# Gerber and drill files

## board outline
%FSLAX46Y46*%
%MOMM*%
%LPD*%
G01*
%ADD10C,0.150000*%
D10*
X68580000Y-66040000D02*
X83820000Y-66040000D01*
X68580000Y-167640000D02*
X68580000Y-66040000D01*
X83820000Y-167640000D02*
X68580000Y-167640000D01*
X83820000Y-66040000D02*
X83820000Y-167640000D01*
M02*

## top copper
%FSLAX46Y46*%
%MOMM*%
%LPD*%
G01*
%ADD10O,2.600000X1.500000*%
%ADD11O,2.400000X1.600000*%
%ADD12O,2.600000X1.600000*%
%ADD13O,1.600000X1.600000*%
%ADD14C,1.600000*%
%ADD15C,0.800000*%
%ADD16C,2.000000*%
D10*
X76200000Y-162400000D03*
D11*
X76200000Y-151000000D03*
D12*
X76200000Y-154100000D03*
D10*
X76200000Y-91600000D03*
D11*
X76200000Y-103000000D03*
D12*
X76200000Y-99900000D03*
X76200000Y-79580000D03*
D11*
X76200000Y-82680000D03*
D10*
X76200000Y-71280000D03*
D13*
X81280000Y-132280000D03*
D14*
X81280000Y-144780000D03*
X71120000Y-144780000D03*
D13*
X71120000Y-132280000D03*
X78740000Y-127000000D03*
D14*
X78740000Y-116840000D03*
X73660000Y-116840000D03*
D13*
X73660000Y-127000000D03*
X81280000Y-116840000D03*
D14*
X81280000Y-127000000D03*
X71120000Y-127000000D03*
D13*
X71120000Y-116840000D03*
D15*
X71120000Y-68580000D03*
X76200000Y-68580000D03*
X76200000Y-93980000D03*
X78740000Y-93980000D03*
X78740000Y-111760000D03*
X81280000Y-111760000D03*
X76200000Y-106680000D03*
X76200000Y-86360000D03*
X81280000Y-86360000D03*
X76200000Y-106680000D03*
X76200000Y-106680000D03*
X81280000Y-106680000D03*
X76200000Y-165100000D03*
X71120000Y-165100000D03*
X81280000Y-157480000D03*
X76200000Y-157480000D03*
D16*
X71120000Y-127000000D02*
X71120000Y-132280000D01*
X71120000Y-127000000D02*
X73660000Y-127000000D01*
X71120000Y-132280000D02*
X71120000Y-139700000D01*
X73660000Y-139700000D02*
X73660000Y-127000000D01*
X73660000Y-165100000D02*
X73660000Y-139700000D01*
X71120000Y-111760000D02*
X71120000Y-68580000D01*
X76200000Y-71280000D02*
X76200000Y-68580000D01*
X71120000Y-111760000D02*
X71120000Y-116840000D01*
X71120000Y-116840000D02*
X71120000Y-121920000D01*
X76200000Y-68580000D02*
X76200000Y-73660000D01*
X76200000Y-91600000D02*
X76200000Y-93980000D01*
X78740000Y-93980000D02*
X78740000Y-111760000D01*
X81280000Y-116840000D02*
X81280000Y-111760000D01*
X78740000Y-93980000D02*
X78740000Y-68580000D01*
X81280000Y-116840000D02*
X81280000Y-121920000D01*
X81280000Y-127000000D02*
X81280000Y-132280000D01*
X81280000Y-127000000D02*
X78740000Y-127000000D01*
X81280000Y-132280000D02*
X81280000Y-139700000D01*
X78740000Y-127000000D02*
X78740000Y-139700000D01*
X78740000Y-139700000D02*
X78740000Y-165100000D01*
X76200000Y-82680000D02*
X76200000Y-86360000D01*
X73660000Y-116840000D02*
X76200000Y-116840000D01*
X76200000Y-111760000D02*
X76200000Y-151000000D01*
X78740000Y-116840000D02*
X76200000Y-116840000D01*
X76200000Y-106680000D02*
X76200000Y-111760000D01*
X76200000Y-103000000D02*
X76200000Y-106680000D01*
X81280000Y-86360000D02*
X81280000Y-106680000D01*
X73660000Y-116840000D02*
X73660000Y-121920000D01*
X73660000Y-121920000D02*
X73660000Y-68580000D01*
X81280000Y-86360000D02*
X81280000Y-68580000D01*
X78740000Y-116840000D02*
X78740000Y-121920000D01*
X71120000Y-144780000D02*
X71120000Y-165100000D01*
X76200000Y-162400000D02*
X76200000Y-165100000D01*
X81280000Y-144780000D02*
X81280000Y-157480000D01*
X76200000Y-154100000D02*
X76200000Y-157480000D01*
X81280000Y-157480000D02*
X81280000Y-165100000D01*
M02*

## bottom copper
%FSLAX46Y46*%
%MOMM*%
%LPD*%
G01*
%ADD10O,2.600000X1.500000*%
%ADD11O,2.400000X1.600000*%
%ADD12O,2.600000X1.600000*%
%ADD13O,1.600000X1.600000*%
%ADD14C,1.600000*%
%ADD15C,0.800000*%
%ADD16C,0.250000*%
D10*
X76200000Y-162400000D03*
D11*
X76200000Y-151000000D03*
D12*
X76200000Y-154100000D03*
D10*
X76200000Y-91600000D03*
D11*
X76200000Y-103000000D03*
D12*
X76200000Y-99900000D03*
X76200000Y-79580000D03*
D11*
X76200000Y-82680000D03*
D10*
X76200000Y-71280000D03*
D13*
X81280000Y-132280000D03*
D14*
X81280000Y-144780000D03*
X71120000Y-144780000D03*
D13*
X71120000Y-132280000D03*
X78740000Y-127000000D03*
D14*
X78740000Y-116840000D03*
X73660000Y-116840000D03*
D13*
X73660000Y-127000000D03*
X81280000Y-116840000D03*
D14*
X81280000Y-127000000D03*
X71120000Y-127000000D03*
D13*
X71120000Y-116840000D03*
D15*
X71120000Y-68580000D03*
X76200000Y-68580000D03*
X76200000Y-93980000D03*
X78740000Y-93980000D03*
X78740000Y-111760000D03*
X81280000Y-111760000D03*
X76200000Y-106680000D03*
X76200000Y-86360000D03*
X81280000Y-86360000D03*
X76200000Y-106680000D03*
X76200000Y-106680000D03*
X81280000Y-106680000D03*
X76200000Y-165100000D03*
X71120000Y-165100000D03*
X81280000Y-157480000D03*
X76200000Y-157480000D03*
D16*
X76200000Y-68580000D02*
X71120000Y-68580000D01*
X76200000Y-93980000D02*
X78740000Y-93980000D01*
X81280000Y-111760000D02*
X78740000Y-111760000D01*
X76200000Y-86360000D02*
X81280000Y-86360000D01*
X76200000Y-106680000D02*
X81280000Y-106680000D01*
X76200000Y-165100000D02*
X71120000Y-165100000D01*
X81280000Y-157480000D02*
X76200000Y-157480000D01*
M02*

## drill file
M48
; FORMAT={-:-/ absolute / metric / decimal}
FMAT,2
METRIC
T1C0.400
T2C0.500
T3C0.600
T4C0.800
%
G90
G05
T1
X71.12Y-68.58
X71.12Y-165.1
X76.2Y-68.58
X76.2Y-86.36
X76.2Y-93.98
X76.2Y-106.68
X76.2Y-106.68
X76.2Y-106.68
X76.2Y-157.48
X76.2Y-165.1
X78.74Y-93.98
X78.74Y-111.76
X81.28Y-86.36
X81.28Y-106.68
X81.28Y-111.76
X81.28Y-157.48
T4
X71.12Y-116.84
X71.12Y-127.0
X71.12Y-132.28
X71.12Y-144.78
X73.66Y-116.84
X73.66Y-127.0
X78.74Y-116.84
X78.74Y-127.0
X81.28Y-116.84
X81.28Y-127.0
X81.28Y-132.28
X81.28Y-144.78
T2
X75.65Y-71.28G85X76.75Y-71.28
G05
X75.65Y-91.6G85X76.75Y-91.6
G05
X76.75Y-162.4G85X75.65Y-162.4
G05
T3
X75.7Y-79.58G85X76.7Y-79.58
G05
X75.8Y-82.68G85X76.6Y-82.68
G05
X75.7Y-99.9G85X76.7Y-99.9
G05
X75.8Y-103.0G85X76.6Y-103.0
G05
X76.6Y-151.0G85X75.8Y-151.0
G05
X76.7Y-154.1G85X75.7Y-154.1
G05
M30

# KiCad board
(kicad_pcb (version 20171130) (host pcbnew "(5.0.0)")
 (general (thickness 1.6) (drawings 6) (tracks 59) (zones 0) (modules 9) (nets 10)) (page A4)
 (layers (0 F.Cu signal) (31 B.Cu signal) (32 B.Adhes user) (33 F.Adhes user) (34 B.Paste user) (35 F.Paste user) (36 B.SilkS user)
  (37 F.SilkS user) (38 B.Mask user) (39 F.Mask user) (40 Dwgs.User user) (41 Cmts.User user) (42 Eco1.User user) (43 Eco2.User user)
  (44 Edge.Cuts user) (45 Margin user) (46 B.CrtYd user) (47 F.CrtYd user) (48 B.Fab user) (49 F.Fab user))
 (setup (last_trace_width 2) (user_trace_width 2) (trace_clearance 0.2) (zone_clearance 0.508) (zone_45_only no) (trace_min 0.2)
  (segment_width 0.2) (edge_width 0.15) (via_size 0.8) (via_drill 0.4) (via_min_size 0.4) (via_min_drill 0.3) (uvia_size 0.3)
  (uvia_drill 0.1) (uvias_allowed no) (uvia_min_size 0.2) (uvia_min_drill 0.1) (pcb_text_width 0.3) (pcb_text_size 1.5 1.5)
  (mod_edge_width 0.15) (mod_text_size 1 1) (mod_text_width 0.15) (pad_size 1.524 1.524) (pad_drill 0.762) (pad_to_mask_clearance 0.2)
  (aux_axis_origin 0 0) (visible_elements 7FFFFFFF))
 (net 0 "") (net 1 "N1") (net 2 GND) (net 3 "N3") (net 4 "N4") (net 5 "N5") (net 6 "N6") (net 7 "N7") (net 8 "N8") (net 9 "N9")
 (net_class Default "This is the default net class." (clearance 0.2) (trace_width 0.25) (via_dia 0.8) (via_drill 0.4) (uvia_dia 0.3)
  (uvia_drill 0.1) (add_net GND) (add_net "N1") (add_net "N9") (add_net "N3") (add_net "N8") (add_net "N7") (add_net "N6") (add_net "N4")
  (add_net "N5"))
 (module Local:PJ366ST (layer F.Cu) (at 76.2 157.48 180)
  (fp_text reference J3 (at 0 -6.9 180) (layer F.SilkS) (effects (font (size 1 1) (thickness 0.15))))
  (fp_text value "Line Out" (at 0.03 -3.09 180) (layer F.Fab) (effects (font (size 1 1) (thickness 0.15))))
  (pad T thru_hole oval (at 0 -4.92 180) (size 2.6 1.5) (drill oval 1.6 0.5) (layers *.Cu *.Mask) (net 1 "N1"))
  (pad S thru_hole oval (at 0 6.48 180) (size 2.4 1.6) (drill oval 1.4 0.6) (layers *.Cu *.Mask) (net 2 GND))
  (pad R thru_hole oval (at 0 3.38 180) (size 2.6 1.6) (drill oval 1.6 0.6) (layers *.Cu *.Mask) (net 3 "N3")))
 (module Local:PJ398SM (layer F.Cu) (at 76.2 96.52)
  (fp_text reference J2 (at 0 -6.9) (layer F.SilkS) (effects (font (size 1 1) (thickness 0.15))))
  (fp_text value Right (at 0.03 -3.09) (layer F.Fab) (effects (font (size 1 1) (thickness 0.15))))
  (pad T thru_hole oval (at 0 -4.92) (size 2.6 1.5) (drill oval 1.6 0.5) (layers *.Cu *.Mask) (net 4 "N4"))
  (pad S thru_hole oval (at 0 6.48) (size 2.4 1.6) (drill oval 1.4 0.6) (layers *.Cu *.Mask) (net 2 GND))
  (pad TN thru_hole oval (at 0 3.38) (size 2.6 1.6) (drill oval 1.6 0.6) (layers *.Cu *.Mask) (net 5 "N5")))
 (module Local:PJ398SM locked (layer F.Cu) (at 76.2 76.2)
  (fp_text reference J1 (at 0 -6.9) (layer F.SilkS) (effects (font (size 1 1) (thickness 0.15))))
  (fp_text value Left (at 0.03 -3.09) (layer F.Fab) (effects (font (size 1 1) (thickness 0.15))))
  (pad TN thru_hole oval (at 0 3.38) (size 2.6 1.6) (drill oval 1.6 0.6) (layers *.Cu *.Mask) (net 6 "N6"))
  (pad S thru_hole oval (at 0 6.48) (size 2.4 1.6) (drill oval 1.4 0.6) (layers *.Cu *.Mask) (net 2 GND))
  (pad T thru_hole oval (at 0 -4.92) (size 2.6 1.5) (drill oval 1.6 0.5) (layers *.Cu *.Mask) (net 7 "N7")))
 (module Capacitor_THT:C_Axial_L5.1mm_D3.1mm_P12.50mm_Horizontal (layer F.Cu) (at 81.28 144.78 90)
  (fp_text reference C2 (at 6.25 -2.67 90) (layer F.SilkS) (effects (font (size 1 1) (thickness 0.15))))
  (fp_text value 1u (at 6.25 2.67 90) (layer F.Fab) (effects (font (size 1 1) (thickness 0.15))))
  (pad 2 thru_hole oval (at 12.5 0 90) (size 1.6 1.6) (drill 0.8) (layers *.Cu *.Mask) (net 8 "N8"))
  (pad 1 thru_hole circle (at 0 0 90) (size 1.6 1.6) (drill 0.8) (layers *.Cu *.Mask) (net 3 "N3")))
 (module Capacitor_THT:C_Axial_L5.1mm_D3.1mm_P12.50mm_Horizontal (layer F.Cu) (at 71.12 144.78 90)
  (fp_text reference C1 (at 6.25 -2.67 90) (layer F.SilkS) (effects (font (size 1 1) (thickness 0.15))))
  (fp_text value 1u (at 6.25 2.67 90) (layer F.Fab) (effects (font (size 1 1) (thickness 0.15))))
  (pad 1 thru_hole circle (at 0 0 90) (size 1.6 1.6) (drill 0.8) (layers *.Cu *.Mask) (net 1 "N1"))
  (pad 2 thru_hole oval (at 12.5 0 90) (size 1.6 1.6) (drill 0.8) (layers *.Cu *.Mask) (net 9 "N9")))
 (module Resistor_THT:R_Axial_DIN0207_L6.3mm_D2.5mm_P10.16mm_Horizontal (layer F.Cu) (at 78.74 116.84 270)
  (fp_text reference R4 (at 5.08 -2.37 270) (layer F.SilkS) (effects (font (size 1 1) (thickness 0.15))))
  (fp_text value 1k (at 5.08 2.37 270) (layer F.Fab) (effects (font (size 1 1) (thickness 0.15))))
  (pad 2 thru_hole oval (at 10.16 0 270) (size 1.6 1.6) (drill 0.8) (layers *.Cu *.Mask) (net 8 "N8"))
  (pad 1 thru_hole circle (at 0 0 270) (size 1.6 1.6) (drill 0.8) (layers *.Cu *.Mask) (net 2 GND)))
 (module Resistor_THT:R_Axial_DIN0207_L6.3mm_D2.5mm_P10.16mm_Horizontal (layer F.Cu) (at 73.66 116.84 270)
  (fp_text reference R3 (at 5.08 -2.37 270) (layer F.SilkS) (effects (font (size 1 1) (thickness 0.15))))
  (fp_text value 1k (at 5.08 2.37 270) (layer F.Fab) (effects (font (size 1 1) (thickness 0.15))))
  (pad 1 thru_hole circle (at 0 0 270) (size 1.6 1.6) (drill 0.8) (layers *.Cu *.Mask) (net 2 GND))
  (pad 2 thru_hole oval (at 10.16 0 270) (size 1.6 1.6) (drill 0.8) (layers *.Cu *.Mask) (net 9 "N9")))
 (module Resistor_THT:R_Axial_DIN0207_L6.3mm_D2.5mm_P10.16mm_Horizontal (layer F.Cu) (at 81.28 127 90)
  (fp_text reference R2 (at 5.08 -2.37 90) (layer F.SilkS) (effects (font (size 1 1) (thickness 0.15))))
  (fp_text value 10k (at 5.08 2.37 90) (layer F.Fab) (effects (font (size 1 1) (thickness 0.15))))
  (pad 2 thru_hole oval (at 10.16 0 90) (size 1.6 1.6) (drill 0.8) (layers *.Cu *.Mask) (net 4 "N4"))
  (pad 1 thru_hole circle (at 0 0 90) (size 1.6 1.6) (drill 0.8) (layers *.Cu *.Mask) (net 8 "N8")))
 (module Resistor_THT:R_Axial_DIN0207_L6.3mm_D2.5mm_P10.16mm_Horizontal (layer F.Cu) (at 71.12 127 90)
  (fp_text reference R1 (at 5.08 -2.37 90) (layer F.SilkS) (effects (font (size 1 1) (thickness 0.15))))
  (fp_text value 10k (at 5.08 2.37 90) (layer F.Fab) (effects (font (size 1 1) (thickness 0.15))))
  (pad 1 thru_hole circle (at 0 0 90) (size 1.6 1.6) (drill 0.8) (layers *.Cu *.Mask) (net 9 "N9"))
  (pad 2 thru_hole oval (at 10.16 0 90) (size 1.6 1.6) (drill 0.8) (layers *.Cu *.Mask) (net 7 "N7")))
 (gr_line (start 68.58 66.04) (end 83.82 66.04) (layer Edge.Cuts) (width 0.15))
 (gr_line (start 68.58 167.64) (end 68.58 66.04) (layer Edge.Cuts) (width 0.15))
 (gr_line (start 83.82 167.64) (end 68.58 167.64) (layer Edge.Cuts) (width 0.15))
 (gr_line (start 83.82 66.04) (end 83.82 167.64) (layer Edge.Cuts) (width 0.15))
 (segment (start 71.12 127) (end 71.12 132.28) (width 2) (layer F.Cu) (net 9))
 (segment (start 71.12 127) (end 73.66 127) (width 2) (layer F.Cu) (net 9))
 (segment (start 71.12 132.28) (end 71.12 139.7) (width 2) (layer F.Cu) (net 9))
 (segment (start 73.66 139.7) (end 73.66 127) (width 2) (layer F.Cu) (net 9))
 (segment (start 73.66 165.1) (end 73.66 139.7) (width 2) (layer F.Cu) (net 9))
 (segment (start 71.12 111.76) (end 71.12 68.58) (width 2) (layer F.Cu) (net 7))
 (via (at 71.12 68.58) (size 0.8) (drill 0.4) (layers F.Cu B.Cu) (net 7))
 (segment (start 76.2 71.28) (end 76.2 68.58) (width 2) (layer F.Cu) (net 7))
 (via (at 76.2 68.58) (size 0.8) (drill 0.4) (layers F.Cu B.Cu) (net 7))
 (segment (start 76.2 68.58) (end 71.12 68.58) (width 0.25) (layer B.Cu) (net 7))
 (segment (start 71.12 111.76) (end 71.12 116.84) (width 2) (layer F.Cu) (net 7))
 (segment (start 71.12 116.84) (end 71.12 121.92) (width 2) (layer F.Cu) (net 7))
 (segment (start 76.2 68.58) (end 76.2 73.66) (width 2) (layer F.Cu) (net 7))
 (segment (start 76.2 91.6) (end 76.2 93.98) (width 2) (layer F.Cu) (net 4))
 (via (at 76.2 93.98) (size 0.8) (drill 0.4) (layers F.Cu B.Cu) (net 4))
 (via (at 78.74 93.98) (size 0.8) (drill 0.4) (layers F.Cu B.Cu) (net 4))
 (segment (start 76.2 93.98) (end 78.74 93.98) (width 0.25) (layer B.Cu) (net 4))
 (segment (start 78.74 93.98) (end 78.74 111.76) (width 2) (layer F.Cu) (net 4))
 (via (at 78.74 111.76) (size 0.8) (drill 0.4) (layers F.Cu B.Cu) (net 4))
 (via (at 81.28 111.76) (size 0.8) (drill 0.4) (layers F.Cu B.Cu) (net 4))
 (segment (start 81.28 116.84) (end 81.28 111.76) (width 2) (layer F.Cu) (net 4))
 (segment (start 81.28 111.76) (end 78.74 111.76) (width 0.25) (layer B.Cu) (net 4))
 (segment (start 78.74 93.98) (end 78.74 68.58) (width 2) (layer F.Cu) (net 4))
 (segment (start 81.28 116.84) (end 81.28 121.92) (width 2) (layer F.Cu) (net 4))
 (segment (start 81.28 127) (end 81.28 132.28) (width 2) (layer F.Cu) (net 8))
 (segment (start 81.28 127) (end 78.74 127) (width 2) (layer F.Cu) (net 8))
 (segment (start 81.28 132.28) (end 81.28 139.7) (width 2) (layer F.Cu) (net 8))
 (segment (start 78.74 127) (end 78.74 139.7) (width 2) (layer F.Cu) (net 8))
 (segment (start 78.74 139.7) (end 78.74 165.1) (width 2) (layer F.Cu) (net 8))
 (segment (start 76.2 82.68) (end 76.2 86.36) (width 2) (layer F.Cu) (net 2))
 (segment (start 73.66 116.84) (end 76.2 116.84) (width 2) (layer F.Cu) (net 2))
 (segment (start 76.2 111.76) (end 76.2 151) (width 2) (layer F.Cu) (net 2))
 (segment (start 78.74 116.84) (end 76.2 116.84) (width 2) (layer F.Cu) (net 2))
 (via (at 76.2 106.68) (size 0.8) (drill 0.4) (layers F.Cu B.Cu) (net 2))
 (segment (start 76.2 106.68) (end 76.2 111.76) (width 2) (layer F.Cu) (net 2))
 (segment (start 76.2 103) (end 76.2 106.68) (width 2) (layer F.Cu) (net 2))
 (via (at 76.2 86.36) (size 0.8) (drill 0.4) (layers F.Cu B.Cu) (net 2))
 (via (at 81.28 86.36) (size 0.8) (drill 0.4) (layers F.Cu B.Cu) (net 2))
 (segment (start 76.2 86.36) (end 81.28 86.36) (width 0.25) (layer B.Cu) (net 2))
 (via (at 76.2 106.68) (size 0.8) (drill 0.4) (layers F.Cu B.Cu) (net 2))
 (via (at 76.2 106.68) (size 0.8) (drill 0.4) (layers F.Cu B.Cu) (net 2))
 (via (at 81.28 106.68) (size 0.8) (drill 0.4) (layers F.Cu B.Cu) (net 2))
 (segment (start 76.2 106.68) (end 81.28 106.68) (width 0.25) (layer B.Cu) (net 2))
 (segment (start 81.28 86.36) (end 81.28 106.68) (width 2) (layer F.Cu) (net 2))
 (segment (start 73.66 116.84) (end 73.66 121.92) (width 2) (layer F.Cu) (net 2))
 (segment (start 73.66 121.92) (end 73.66 68.58) (width 2) (layer F.Cu) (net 2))
 (segment (start 81.28 86.36) (end 81.28 68.58) (width 2) (layer F.Cu) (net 2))
 (segment (start 78.74 116.84) (end 78.74 121.92) (width 2) (layer F.Cu) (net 2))
 (segment (start 71.12 144.78) (end 71.12 165.1) (width 2) (layer F.Cu) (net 1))
 (segment (start 76.2 162.4) (end 76.2 165.1) (width 2) (layer F.Cu) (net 1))
 (via (at 76.2 165.1) (size 0.8) (drill 0.4) (layers F.Cu B.Cu) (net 1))
 (via (at 71.12 165.1) (size 0.8) (drill 0.4) (layers F.Cu B.Cu) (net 1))
 (segment (start 76.2 165.1) (end 71.12 165.1) (width 0.25) (layer B.Cu) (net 1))
 (segment (start 81.28 144.78) (end 81.28 157.48) (width 2) (layer F.Cu) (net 3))
 (via (at 81.28 157.48) (size 0.8) (drill 0.4) (layers F.Cu B.Cu) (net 3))
 (segment (start 76.2 154.1) (end 76.2 157.48) (width 2) (layer F.Cu) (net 3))
 (via (at 76.2 157.48) (size 0.8) (drill 0.4) (layers F.Cu B.Cu) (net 3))
 (segment (start 81.28 157.48) (end 76.2 157.48) (width 0.25) (layer B.Cu) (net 3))
 (segment (start 81.28 157.48) (end 81.28 165.1) (width 2) (layer F.Cu) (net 3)))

